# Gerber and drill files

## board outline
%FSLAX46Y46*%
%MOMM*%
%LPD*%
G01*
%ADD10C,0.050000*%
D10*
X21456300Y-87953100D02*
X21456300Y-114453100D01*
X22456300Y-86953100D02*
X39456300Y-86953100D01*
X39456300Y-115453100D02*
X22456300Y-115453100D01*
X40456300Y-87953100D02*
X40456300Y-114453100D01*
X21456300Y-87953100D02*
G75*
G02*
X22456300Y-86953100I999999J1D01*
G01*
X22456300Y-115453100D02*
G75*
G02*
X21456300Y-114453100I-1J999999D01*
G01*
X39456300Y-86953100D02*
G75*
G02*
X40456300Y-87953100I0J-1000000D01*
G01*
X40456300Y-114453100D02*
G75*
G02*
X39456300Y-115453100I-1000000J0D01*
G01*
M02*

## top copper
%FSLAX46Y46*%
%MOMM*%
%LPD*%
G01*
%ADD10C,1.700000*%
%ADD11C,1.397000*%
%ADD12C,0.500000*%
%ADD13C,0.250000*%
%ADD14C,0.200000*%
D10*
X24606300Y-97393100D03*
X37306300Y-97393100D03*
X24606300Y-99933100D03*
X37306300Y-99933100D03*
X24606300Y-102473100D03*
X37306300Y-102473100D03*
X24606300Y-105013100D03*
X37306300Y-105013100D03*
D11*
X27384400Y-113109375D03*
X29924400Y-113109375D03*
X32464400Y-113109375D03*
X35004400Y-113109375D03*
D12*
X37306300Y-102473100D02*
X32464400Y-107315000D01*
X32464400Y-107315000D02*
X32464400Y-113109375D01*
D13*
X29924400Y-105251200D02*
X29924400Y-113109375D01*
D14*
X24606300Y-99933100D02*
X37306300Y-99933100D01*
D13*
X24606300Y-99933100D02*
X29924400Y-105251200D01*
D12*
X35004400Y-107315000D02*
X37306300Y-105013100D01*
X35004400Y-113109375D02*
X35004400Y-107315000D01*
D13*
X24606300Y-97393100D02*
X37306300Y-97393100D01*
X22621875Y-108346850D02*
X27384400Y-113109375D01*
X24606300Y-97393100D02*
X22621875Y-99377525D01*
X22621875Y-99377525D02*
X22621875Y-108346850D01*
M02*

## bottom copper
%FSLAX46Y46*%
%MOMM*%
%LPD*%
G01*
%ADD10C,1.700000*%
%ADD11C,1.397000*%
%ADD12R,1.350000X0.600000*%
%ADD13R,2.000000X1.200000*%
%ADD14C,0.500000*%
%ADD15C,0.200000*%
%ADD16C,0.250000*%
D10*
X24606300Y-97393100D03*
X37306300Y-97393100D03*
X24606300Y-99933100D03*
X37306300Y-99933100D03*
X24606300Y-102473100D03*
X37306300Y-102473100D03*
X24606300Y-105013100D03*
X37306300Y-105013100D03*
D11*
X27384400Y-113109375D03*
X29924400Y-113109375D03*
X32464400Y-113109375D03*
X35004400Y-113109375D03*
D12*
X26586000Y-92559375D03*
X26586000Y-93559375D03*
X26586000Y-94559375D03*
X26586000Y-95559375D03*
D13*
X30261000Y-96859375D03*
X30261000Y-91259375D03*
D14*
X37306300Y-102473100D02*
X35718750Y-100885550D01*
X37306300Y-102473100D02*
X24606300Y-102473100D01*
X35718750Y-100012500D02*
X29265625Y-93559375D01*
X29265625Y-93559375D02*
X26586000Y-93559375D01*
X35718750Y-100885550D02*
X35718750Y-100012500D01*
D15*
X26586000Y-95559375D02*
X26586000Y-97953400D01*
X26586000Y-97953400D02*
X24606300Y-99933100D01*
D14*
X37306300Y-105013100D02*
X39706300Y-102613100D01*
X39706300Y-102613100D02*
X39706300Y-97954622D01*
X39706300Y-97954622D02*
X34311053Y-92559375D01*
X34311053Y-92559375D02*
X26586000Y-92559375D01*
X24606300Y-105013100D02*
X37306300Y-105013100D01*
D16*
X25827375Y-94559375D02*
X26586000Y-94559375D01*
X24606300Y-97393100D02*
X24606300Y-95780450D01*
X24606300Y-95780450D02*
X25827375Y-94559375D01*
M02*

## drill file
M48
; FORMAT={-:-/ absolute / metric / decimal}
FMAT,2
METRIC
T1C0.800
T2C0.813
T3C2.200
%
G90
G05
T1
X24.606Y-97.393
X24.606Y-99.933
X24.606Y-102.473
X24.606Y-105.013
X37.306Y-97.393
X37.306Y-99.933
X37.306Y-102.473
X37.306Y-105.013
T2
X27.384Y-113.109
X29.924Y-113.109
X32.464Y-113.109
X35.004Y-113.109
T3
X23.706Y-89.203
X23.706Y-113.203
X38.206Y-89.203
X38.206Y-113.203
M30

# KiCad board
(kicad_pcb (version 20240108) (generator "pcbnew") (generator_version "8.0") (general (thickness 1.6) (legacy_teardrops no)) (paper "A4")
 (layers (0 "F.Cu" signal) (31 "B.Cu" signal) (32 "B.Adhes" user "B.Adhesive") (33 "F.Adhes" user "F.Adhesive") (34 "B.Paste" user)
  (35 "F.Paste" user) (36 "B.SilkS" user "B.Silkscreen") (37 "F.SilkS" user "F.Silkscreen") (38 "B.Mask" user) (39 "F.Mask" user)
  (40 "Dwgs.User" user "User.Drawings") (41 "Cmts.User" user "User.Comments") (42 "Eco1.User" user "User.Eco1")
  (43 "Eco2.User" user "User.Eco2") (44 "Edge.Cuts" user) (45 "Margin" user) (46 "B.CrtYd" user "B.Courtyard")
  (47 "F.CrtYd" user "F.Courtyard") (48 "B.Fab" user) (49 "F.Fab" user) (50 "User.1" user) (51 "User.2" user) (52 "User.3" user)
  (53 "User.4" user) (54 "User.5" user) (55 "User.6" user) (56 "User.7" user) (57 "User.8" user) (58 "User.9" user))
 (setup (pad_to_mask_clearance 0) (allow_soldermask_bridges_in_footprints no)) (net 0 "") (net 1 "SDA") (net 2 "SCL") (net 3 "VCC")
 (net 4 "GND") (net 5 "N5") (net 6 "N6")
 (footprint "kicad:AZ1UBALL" (layer "F.Cu") (at 30.9563 101.2031)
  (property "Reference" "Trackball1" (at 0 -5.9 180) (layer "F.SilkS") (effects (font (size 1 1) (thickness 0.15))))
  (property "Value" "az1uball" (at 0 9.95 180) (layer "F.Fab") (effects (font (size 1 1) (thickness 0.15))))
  (pad "1" thru_hole circle (at -6.35 -3.81) (size 1.7 1.7) (drill 0.8) (layers "*.Cu" "*.Mask") (remove_unused_layers no) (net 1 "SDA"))
  (pad "1" thru_hole circle (at 6.35 -3.81) (size 1.7 1.7) (drill 0.8) (layers "*.Cu" "*.Mask") (remove_unused_layers no) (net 1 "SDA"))
  (pad "2" thru_hole circle (at -6.35 -1.27) (size 1.7 1.7) (drill 0.8) (layers "*.Cu" "*.Mask") (remove_unused_layers no) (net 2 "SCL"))
  (pad "2" thru_hole circle (at 6.35 -1.27) (size 1.7 1.7) (drill 0.8) (layers "*.Cu" "*.Mask") (remove_unused_layers no) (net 2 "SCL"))
  (pad "3" thru_hole circle (at -6.35 1.27) (size 1.7 1.7) (drill 0.8) (layers "*.Cu" "*.Mask") (remove_unused_layers no) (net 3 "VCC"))
  (pad "3" thru_hole circle (at 6.35 1.27) (size 1.7 1.7) (drill 0.8) (layers "*.Cu" "*.Mask") (remove_unused_layers no) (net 3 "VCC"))
  (pad "4" thru_hole circle (at -6.35 3.81) (size 1.7 1.7) (drill 0.8) (layers "*.Cu" "*.Mask") (remove_unused_layers no) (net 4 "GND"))
  (pad "4" thru_hole circle (at 6.35 3.81) (size 1.7 1.7) (drill 0.8) (layers "*.Cu" "*.Mask") (remove_unused_layers no) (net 4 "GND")))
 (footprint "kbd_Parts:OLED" (layer "F.Cu") (at 27.3844 113.109375)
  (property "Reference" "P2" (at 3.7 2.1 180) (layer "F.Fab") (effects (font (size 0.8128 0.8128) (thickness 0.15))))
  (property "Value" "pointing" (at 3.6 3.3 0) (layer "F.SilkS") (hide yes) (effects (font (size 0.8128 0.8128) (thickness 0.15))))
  (pad "1" thru_hole circle (at 0 0) (size 1.397 1.397) (drill 0.8128) (layers "*.Cu" "*.Mask" "F.SilkS") (remove_unused_layers no)
   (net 1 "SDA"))
  (pad "2" thru_hole circle (at 2.54 0) (size 1.397 1.397) (drill 0.8128) (layers "*.Cu" "*.Mask" "F.SilkS") (remove_unused_layers no)
   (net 2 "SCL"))
  (pad "3" thru_hole circle (at 5.08 0) (size 1.397 1.397) (drill 0.8128) (layers "*.Cu" "*.Mask" "F.SilkS") (remove_unused_layers no)
   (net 3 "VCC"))
  (pad "4" thru_hole circle (at 7.62 0) (size 1.397 1.397) (drill 0.8128) (layers "*.Cu" "*.Mask" "F.SilkS") (remove_unused_layers no)
   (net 4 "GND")))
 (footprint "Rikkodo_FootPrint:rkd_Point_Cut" (layer "F.Cu") (at 30.9563 101.2031)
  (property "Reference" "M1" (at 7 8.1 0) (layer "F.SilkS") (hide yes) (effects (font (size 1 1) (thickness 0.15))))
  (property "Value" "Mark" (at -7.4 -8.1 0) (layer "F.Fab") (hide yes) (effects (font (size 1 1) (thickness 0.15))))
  (fp_line (start -9.5 -13.25) (end -9.5 13.25) (stroke (width 0.05) (type default)) (layer "Edge.Cuts"))
  (fp_line (start -8.5 -14.25) (end 8.5 -14.25) (stroke (width 0.05) (type default)) (layer "Edge.Cuts"))
  (fp_line (start 8.5 14.25) (end -8.5 14.25) (stroke (width 0.05) (type default)) (layer "Edge.Cuts"))
  (fp_line (start 9.5 -13.25) (end 9.5 13.25) (stroke (width 0.05) (type default)) (layer "Edge.Cuts"))
  (fp_arc (start -9.5 -13.25) (mid -9.207107 -13.957107) (end -8.5 -14.25) (stroke (width 0.05) (type default)) (layer "Edge.Cuts"))
  (fp_arc (start -8.5 14.25) (mid -9.207107 13.957107) (end -9.5 13.25) (stroke (width 0.05) (type default)) (layer "Edge.Cuts"))
  (fp_arc (start 8.5 -14.25) (mid 9.207107 -13.957107) (end 9.5 -13.25) (stroke (width 0.05) (type default)) (layer "Edge.Cuts"))
  (fp_arc (start 9.5 13.25) (mid 9.207107 13.957107) (end 8.5 14.25) (stroke (width 0.05) (type default)) (layer "Edge.Cuts"))
  (pad "" np_thru_hole circle (at -7.25 -12) (size 2.2 2.2) (drill 2.2) (layers "*.Cu" "*.Mask"))
  (pad "" np_thru_hole circle (at -7.25 12) (size 2.2 2.2) (drill 2.2) (layers "*.Cu" "*.Mask"))
  (pad "" np_thru_hole circle (at 7.25 -12) (size 2.2 2.2) (drill 2.2) (layers "*.Cu" "*.Mask"))
  (pad "" np_thru_hole circle (at 7.25 12) (size 2.2 2.2) (drill 2.2) (layers "*.Cu" "*.Mask")))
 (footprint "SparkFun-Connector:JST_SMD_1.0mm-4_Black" (layer "B.Cu") (at 26.586 94.059375 -90)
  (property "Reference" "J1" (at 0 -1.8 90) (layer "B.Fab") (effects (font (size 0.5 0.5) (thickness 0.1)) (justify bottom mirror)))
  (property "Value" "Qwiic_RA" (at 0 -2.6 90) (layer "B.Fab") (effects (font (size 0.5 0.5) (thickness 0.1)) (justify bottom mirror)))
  (pad "1" smd rect (at -1.5 0 270) (size 0.6 1.35) (layers "B.Cu" "B.Paste" "B.Mask") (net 4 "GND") (thermal_bridge_angle 0))
  (pad "2" smd rect (at -0.5 0 270) (size 0.6 1.35) (layers "B.Cu" "B.Paste" "B.Mask") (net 3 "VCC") (thermal_bridge_angle 0))
  (pad "3" smd rect (at 0.5 0 270) (size 0.6 1.35) (layers "B.Cu" "B.Paste" "B.Mask") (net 1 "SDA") (thermal_bridge_angle 0))
  (pad "4" smd rect (at 1.5 0 270) (size 0.6 1.35) (layers "B.Cu" "B.Paste" "B.Mask") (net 2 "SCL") (thermal_bridge_angle 0))
  (pad "NC1" smd rect (at 2.8 -3.675 270) (size 1.2 2) (layers "B.Cu" "B.Paste" "B.Mask") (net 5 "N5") (thermal_bridge_angle 0))
  (pad "NC2" smd rect (at -2.8 -3.675 270) (size 1.2 2) (layers "B.Cu" "B.Paste" "B.Mask") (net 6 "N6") (thermal_bridge_angle 0)))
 (segment (start 37.3063 102.4731) (end 32.4644 107.315) (width 0.5) (layer "F.Cu") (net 3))
 (segment (start 32.4644 107.315) (end 32.4644 113.109375) (width 0.5) (layer "F.Cu") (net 3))
 (segment (start 37.3063 102.4731) (end 35.71875 100.88555) (width 0.5) (layer "B.Cu") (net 3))
 (segment (start 37.3063 102.4731) (end 24.6063 102.4731) (width 0.5) (layer "B.Cu") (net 3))
 (segment (start 35.71875 100.0125) (end 29.265625 93.559375) (width 0.5) (layer "B.Cu") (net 3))
 (segment (start 29.265625 93.559375) (end 26.586 93.559375) (width 0.5) (layer "B.Cu") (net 3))
 (segment (start 35.71875 100.88555) (end 35.71875 100.0125) (width 0.5) (layer "B.Cu") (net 3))
 (segment (start 29.9244 105.2512) (end 29.9244 113.109375) (width 0.25) (layer "F.Cu") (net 2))
 (segment (start 24.6063 99.9331) (end 37.3063 99.9331) (width 0.2) (layer "F.Cu") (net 2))
 (segment (start 24.6063 99.9331) (end 29.9244 105.2512) (width 0.25) (layer "F.Cu") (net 2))
 (segment (start 26.586 95.559375) (end 26.586 97.9534) (width 0.2) (layer "B.Cu") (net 2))
 (segment (start 26.586 97.9534) (end 24.6063 99.9331) (width 0.2) (layer "B.Cu") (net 2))
 (segment (start 35.0044 107.315) (end 37.3063 105.0131) (width 0.5) (layer "F.Cu") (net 4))
 (segment (start 35.0044 113.109375) (end 35.0044 107.315) (width 0.5) (layer "F.Cu") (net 4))
 (segment (start 37.3063 105.0131) (end 39.7063 102.6131) (width 0.5) (layer "B.Cu") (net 4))
 (segment (start 39.7063 102.6131) (end 39.7063 97.954622) (width 0.5) (layer "B.Cu") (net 4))
 (segment (start 39.7063 97.954622) (end 34.311053 92.559375) (width 0.5) (layer "B.Cu") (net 4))
 (segment (start 34.311053 92.559375) (end 26.586 92.559375) (width 0.5) (layer "B.Cu") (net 4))
 (segment (start 24.6063 105.0131) (end 37.3063 105.0131) (width 0.5) (layer "B.Cu") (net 4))
 (segment (start 24.6063 97.3931) (end 37.3063 97.3931) (width 0.25) (layer "F.Cu") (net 1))
 (segment (start 22.621875 108.34685) (end 27.3844 113.109375) (width 0.25) (layer "F.Cu") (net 1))
 (segment (start 24.6063 97.3931) (end 22.621875 99.377525) (width 0.25) (layer "F.Cu") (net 1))
 (segment (start 22.621875 99.377525) (end 22.621875 108.34685) (width 0.25) (layer "F.Cu") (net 1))
 (segment (start 25.827375 94.559375) (end 26.586 94.559375) (width 0.25) (layer "B.Cu") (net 1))
 (segment (start 24.6063 97.3931) (end 24.6063 95.78045) (width 0.25) (layer "B.Cu") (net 1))
 (segment (start 24.6063 95.78045) (end 25.827375 94.559375) (width 0.25) (layer "B.Cu") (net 1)))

